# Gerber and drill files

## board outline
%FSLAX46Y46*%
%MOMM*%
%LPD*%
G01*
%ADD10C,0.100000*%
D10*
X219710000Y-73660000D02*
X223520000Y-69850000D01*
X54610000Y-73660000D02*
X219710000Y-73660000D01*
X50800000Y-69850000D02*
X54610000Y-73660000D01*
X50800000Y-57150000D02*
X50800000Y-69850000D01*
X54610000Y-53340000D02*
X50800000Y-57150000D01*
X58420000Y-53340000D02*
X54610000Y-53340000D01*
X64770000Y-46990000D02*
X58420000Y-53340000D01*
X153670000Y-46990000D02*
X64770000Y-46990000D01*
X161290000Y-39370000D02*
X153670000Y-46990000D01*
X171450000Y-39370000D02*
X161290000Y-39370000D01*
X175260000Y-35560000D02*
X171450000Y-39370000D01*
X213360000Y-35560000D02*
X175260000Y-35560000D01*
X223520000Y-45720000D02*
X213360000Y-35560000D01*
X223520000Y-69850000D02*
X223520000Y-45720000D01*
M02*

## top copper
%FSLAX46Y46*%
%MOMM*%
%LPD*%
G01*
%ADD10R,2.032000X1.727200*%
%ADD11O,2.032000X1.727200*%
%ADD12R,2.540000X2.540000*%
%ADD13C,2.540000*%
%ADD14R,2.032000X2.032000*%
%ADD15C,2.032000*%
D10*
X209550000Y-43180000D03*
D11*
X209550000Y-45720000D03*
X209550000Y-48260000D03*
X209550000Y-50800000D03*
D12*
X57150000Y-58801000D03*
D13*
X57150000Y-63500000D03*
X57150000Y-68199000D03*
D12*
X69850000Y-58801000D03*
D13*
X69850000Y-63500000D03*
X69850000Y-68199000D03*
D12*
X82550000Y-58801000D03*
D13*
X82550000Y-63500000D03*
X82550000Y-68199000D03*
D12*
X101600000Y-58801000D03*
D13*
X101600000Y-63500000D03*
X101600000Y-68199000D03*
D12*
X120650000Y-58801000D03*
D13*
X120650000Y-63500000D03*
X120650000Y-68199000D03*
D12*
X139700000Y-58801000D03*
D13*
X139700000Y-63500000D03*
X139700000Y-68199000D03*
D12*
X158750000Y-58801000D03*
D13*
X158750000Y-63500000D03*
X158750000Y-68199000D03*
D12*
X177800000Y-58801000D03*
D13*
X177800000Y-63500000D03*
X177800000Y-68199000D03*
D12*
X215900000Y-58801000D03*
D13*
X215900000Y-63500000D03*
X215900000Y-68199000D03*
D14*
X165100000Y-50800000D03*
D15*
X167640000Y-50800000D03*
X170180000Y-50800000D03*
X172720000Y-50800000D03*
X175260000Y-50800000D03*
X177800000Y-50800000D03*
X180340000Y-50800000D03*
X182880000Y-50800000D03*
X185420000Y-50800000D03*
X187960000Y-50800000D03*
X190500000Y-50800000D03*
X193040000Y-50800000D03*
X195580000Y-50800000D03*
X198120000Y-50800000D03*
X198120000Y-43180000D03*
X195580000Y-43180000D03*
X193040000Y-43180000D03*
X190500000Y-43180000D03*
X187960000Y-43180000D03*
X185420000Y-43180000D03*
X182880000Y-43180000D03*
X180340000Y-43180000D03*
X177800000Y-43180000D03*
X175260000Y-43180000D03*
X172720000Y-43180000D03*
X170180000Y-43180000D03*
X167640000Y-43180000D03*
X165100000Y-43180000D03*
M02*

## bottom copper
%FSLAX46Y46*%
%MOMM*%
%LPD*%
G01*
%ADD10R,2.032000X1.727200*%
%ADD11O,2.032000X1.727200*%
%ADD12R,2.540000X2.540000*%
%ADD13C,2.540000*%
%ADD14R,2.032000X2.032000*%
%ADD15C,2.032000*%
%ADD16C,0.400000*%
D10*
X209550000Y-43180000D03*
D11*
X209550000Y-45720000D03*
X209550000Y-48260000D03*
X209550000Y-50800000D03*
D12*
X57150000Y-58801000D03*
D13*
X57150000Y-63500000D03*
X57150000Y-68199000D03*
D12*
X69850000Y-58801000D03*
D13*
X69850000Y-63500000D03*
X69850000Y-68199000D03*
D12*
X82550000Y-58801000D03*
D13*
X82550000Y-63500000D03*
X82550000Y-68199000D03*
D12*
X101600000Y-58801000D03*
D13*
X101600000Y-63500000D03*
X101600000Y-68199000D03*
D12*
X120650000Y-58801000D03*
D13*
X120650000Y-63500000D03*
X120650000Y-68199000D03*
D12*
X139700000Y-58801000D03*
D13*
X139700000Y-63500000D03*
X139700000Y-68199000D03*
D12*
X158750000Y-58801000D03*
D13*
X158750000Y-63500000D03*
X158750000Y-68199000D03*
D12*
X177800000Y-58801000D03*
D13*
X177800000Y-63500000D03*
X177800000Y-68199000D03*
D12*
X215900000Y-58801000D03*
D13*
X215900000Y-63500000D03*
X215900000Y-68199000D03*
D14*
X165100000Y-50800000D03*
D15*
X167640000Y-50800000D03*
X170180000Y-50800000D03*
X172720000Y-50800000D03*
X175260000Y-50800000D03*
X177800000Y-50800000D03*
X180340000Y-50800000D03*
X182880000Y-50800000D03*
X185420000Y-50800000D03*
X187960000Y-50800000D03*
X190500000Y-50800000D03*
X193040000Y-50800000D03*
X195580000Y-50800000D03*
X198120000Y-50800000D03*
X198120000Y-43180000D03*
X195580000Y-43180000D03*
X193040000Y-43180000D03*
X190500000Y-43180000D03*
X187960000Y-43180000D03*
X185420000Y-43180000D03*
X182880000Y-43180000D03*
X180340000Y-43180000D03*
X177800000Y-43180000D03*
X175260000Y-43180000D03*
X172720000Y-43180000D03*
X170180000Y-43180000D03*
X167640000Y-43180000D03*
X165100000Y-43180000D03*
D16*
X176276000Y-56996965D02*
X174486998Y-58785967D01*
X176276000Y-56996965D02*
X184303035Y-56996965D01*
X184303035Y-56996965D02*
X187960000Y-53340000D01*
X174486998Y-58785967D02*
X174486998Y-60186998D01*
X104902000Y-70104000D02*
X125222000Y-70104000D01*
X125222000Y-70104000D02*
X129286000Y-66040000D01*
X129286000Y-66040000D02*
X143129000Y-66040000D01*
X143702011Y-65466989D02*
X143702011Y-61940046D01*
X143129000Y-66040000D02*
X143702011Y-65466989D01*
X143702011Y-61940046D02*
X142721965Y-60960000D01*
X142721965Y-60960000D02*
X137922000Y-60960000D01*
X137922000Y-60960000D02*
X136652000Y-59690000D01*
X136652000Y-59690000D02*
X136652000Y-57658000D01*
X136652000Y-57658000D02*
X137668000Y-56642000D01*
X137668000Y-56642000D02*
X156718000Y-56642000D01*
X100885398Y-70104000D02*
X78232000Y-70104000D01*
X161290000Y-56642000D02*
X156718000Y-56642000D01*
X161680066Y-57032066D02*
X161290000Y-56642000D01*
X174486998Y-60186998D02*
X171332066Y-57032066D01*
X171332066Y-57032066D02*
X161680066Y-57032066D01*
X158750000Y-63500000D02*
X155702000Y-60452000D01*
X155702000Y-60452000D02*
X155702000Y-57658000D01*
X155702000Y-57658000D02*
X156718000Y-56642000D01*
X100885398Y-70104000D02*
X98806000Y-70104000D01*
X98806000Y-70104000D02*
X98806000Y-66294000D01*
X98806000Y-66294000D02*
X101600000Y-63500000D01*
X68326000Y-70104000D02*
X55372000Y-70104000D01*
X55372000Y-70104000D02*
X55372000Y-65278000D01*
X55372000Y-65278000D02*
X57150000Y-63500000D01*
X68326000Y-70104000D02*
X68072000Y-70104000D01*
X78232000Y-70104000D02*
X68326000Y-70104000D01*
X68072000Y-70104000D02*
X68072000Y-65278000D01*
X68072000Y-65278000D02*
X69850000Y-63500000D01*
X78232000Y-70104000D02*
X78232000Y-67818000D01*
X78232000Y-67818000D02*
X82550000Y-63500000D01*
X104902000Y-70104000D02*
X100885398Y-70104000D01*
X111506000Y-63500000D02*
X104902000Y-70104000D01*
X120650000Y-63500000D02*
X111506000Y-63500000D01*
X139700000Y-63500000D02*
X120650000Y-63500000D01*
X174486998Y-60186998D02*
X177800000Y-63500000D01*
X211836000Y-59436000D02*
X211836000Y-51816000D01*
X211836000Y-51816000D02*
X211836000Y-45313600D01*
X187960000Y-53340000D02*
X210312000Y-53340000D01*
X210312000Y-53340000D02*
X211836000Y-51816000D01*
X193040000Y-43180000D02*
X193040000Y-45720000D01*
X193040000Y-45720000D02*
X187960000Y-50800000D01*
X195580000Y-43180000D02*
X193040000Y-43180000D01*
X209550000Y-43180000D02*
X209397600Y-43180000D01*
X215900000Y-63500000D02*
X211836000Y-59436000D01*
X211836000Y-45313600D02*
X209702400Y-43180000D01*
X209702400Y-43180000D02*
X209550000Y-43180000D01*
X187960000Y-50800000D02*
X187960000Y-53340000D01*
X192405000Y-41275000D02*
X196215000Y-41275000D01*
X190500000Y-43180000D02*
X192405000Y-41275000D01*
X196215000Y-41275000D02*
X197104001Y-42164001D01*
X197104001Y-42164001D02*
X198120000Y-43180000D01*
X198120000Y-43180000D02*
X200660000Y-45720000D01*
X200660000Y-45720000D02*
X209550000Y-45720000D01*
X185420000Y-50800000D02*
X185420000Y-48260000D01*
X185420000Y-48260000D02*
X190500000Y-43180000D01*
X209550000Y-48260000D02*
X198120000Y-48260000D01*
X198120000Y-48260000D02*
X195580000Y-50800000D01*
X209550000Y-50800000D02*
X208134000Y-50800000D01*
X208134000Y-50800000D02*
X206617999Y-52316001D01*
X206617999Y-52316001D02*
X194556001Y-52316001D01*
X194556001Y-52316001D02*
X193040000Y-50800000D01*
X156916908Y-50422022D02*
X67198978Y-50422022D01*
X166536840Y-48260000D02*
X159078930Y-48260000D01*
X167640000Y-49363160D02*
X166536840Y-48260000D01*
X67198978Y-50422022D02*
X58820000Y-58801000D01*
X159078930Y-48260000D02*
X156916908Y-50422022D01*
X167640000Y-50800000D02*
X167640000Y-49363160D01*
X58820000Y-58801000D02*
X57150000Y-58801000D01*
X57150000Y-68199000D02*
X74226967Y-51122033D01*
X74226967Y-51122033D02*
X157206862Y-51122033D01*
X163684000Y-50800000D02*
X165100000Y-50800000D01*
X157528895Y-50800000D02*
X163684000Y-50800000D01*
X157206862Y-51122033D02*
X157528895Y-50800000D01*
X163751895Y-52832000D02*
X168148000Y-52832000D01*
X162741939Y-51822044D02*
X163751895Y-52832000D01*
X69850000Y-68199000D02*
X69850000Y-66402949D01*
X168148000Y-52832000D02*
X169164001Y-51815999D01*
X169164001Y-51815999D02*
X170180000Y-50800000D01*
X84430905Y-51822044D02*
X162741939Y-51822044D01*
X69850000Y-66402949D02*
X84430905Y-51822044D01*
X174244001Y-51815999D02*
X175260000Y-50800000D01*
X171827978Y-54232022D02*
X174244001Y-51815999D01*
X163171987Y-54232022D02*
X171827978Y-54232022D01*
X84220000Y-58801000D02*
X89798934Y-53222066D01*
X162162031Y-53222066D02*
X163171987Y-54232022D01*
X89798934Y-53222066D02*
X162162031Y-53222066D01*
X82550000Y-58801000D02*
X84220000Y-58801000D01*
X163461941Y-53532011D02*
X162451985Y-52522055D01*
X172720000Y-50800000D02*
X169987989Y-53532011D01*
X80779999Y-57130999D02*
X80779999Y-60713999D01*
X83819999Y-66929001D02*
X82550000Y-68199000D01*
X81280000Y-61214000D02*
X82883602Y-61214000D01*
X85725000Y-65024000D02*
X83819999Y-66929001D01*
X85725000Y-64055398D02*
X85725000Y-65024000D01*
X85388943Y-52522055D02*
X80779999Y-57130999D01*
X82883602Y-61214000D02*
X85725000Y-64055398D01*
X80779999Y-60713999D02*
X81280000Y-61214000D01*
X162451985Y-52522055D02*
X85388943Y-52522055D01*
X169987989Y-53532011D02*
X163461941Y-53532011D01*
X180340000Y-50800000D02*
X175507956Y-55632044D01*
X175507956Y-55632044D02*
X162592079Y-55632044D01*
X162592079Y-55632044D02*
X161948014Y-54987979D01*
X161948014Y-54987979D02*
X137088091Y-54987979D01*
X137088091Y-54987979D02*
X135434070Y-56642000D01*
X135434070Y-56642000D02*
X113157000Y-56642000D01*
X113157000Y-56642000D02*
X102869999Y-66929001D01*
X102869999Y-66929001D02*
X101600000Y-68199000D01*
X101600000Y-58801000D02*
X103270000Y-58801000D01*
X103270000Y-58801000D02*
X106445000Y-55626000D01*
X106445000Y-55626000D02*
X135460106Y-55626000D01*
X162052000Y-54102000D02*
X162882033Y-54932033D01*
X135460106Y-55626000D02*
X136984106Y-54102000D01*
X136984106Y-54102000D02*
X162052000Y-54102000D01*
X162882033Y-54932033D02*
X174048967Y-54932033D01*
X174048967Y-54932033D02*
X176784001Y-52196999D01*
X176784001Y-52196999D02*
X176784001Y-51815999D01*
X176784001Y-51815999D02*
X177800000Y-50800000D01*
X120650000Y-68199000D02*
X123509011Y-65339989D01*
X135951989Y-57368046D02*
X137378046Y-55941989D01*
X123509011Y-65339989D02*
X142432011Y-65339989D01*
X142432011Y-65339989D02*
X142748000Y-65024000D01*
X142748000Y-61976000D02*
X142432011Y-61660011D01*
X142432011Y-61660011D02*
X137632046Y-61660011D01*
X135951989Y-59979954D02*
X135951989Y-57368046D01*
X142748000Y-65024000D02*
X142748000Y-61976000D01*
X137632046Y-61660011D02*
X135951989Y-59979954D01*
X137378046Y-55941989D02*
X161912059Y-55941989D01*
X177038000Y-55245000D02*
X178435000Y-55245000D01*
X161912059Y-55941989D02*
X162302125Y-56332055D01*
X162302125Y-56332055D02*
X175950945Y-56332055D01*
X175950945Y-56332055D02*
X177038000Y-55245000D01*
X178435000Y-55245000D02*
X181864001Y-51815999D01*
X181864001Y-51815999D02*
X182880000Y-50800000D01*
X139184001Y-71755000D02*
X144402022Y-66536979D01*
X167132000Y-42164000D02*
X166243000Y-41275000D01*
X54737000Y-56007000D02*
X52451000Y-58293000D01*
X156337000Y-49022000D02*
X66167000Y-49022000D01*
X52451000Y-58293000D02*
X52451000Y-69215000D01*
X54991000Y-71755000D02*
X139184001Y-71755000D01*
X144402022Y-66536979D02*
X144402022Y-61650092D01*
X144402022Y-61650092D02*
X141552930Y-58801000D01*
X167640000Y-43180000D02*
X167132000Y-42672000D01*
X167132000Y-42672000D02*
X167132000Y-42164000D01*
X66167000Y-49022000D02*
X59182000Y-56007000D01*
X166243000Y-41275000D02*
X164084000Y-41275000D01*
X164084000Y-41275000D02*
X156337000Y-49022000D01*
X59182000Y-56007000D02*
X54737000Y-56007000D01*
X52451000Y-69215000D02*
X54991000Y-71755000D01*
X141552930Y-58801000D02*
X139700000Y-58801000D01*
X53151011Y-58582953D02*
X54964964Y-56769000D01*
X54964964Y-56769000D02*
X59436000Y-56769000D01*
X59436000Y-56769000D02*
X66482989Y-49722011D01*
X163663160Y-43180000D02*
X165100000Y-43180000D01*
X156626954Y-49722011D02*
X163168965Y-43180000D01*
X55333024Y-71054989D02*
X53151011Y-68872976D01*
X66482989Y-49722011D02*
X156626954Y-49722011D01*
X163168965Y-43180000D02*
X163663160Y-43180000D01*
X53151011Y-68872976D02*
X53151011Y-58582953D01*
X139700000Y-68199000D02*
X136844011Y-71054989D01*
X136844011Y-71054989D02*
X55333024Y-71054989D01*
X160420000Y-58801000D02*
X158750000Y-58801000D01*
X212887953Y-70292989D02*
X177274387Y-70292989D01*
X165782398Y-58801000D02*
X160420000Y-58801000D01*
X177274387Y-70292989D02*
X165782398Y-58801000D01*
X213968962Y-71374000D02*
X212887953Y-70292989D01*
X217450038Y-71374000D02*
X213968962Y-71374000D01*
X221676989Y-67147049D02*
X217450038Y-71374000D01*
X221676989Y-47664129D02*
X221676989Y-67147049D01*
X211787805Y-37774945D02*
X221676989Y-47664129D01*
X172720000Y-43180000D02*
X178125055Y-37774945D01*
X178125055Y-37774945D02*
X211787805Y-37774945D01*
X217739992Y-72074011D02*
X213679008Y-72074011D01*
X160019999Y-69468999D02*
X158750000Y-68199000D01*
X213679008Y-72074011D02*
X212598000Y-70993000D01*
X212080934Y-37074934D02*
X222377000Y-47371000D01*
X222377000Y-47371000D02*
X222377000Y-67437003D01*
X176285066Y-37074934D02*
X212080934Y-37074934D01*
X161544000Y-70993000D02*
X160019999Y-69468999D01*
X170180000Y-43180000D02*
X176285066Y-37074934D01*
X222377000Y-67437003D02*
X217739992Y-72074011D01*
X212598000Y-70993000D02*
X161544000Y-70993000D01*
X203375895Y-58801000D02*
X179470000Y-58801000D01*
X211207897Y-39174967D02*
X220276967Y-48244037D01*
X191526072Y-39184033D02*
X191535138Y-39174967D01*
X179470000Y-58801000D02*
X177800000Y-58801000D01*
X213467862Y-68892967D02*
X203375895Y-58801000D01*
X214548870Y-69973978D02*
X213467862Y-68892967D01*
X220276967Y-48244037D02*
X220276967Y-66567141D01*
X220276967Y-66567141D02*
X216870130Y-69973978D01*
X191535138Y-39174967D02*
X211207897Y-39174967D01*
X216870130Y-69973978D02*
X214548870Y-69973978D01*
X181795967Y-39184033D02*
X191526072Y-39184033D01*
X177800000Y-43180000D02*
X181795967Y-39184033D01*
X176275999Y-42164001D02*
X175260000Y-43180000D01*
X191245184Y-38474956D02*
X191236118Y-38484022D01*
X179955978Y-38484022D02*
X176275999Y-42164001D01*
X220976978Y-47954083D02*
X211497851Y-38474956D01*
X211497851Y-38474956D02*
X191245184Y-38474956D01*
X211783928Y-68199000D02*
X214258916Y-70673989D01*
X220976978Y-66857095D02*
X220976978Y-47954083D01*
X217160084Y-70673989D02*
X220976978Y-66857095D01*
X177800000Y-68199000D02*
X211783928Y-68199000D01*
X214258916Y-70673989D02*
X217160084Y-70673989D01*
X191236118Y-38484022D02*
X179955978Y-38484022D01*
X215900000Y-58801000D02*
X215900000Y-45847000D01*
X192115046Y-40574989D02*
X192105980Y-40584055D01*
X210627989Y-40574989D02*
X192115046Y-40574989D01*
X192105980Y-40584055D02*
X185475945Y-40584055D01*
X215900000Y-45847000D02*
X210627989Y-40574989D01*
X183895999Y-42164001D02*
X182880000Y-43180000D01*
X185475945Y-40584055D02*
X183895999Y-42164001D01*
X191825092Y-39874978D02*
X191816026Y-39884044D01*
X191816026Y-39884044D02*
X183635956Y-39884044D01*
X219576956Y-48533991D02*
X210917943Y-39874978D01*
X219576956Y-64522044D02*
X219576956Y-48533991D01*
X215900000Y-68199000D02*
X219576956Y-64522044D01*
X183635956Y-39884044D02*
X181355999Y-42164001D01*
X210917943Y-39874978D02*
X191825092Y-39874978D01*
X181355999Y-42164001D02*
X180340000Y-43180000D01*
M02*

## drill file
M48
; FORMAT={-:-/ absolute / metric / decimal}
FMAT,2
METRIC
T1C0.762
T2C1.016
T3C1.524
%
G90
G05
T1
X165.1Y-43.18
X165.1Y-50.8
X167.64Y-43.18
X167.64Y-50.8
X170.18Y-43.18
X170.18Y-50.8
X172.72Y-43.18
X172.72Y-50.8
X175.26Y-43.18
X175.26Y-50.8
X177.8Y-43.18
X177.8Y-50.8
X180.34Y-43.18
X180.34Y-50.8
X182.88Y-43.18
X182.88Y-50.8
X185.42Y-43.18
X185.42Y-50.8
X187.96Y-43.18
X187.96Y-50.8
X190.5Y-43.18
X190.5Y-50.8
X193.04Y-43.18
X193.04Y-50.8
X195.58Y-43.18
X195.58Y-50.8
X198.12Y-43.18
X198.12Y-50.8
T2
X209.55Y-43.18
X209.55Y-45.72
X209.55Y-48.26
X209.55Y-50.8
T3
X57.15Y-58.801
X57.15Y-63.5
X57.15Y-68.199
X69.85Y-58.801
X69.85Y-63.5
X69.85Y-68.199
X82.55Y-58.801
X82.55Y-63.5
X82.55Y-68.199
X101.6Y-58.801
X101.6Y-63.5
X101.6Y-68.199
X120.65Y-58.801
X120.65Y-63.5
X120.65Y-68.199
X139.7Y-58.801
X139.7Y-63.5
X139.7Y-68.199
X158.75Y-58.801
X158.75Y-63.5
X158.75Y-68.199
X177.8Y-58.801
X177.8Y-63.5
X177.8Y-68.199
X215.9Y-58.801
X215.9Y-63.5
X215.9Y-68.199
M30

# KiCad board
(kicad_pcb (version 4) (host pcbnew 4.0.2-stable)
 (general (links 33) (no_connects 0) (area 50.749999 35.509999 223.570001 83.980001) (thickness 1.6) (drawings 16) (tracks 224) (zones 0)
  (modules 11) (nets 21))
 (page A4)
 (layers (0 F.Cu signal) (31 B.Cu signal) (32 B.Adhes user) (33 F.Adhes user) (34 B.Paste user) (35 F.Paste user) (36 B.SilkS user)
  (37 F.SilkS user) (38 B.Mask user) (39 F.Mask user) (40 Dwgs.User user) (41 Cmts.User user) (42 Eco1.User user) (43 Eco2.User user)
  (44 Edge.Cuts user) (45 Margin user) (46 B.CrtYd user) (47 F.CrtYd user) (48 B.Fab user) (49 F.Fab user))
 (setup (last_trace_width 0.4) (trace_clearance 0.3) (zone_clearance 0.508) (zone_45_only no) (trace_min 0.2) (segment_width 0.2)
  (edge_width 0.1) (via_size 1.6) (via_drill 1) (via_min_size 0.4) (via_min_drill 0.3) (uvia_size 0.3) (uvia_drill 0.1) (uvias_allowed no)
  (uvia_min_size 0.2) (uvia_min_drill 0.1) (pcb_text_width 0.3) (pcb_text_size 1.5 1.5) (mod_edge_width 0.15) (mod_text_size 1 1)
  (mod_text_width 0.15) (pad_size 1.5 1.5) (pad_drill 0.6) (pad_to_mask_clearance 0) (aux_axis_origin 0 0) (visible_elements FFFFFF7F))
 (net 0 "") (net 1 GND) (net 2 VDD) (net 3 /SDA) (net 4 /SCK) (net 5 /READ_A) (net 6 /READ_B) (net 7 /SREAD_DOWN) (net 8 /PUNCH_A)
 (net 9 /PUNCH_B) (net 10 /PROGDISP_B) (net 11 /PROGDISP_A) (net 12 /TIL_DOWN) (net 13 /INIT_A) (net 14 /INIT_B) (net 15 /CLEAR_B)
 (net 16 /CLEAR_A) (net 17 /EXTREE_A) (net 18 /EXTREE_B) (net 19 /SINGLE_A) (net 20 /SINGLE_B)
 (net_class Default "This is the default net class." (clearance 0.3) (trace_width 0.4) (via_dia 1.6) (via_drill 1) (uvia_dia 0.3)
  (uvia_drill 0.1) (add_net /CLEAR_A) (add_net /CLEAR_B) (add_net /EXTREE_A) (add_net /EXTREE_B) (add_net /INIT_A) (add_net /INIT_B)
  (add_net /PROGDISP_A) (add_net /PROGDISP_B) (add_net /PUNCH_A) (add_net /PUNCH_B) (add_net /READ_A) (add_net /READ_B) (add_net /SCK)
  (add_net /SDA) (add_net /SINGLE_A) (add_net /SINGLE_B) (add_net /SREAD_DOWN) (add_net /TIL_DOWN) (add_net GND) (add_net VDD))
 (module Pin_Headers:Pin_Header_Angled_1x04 (layer F.Cu) (at 209.55 43.18)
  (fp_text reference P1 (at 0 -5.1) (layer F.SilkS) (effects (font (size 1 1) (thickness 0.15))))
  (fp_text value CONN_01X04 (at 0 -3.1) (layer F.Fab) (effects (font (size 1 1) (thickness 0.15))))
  (pad 1 thru_hole rect (at 0 0) (size 2.032 1.7272) (drill 1.016) (layers *.Cu *.Mask F.SilkS) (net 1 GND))
  (pad 2 thru_hole oval (at 0 2.54) (size 2.032 1.7272) (drill 1.016) (layers *.Cu *.Mask F.SilkS) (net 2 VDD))
  (pad 3 thru_hole oval (at 0 5.08) (size 2.032 1.7272) (drill 1.016) (layers *.Cu *.Mask F.SilkS) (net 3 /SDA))
  (pad 4 thru_hole oval (at 0 7.62) (size 2.032 1.7272) (drill 1.016) (layers *.Cu *.Mask F.SilkS) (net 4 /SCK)))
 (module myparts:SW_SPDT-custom (layer F.Cu) (at 57.15 63.5 270)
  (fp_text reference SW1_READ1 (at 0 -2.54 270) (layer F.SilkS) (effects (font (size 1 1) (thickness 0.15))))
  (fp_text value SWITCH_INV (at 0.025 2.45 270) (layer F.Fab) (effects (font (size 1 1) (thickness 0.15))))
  (pad 1 thru_hole rect (at -4.699 0 270) (size 2.54 2.54) (drill 1.524) (layers *.Cu *.Mask F.SilkS) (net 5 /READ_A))
  (pad 2 thru_hole circle (at 0 0 270) (size 2.54 2.54) (drill 1.524) (layers *.Cu *.Mask F.SilkS) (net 1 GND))
  (pad 3 thru_hole circle (at 4.699 0 270) (size 2.54 2.54) (drill 1.524) (layers *.Cu *.Mask F.SilkS) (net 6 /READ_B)))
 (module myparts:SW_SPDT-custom (layer F.Cu) (at 69.85 63.5 270)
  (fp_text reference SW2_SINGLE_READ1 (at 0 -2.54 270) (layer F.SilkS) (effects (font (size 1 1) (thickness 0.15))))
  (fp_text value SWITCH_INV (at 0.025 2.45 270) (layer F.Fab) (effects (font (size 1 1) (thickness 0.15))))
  (pad 1 thru_hole rect (at -4.699 0 270) (size 2.54 2.54) (drill 1.524) (layers *.Cu *.Mask F.SilkS))
  (pad 2 thru_hole circle (at 0 0 270) (size 2.54 2.54) (drill 1.524) (layers *.Cu *.Mask F.SilkS) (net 1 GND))
  (pad 3 thru_hole circle (at 4.699 0 270) (size 2.54 2.54) (drill 1.524) (layers *.Cu *.Mask F.SilkS) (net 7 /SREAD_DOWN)))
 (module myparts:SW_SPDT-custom (layer F.Cu) (at 82.55 63.5 270)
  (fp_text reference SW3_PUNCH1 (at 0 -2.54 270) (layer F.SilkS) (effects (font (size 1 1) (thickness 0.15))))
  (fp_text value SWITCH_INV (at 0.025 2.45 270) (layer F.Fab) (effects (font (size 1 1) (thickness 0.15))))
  (pad 1 thru_hole rect (at -4.699 0 270) (size 2.54 2.54) (drill 1.524) (layers *.Cu *.Mask F.SilkS) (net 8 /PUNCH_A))
  (pad 2 thru_hole circle (at 0 0 270) (size 2.54 2.54) (drill 1.524) (layers *.Cu *.Mask F.SilkS) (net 1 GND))
  (pad 3 thru_hole circle (at 4.699 0 270) (size 2.54 2.54) (drill 1.524) (layers *.Cu *.Mask F.SilkS) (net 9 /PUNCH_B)))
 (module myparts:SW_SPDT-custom (layer F.Cu) (at 101.6 63.5 270)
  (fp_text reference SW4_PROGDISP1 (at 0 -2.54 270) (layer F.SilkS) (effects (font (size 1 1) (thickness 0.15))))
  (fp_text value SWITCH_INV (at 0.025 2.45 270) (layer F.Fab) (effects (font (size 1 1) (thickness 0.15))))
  (pad 1 thru_hole rect (at -4.699 0 270) (size 2.54 2.54) (drill 1.524) (layers *.Cu *.Mask F.SilkS) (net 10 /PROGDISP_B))
  (pad 2 thru_hole circle (at 0 0 270) (size 2.54 2.54) (drill 1.524) (layers *.Cu *.Mask F.SilkS) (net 1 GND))
  (pad 3 thru_hole circle (at 4.699 0 270) (size 2.54 2.54) (drill 1.524) (layers *.Cu *.Mask F.SilkS) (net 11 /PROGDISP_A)))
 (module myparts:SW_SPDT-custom (layer F.Cu) (at 120.65 63.5 270)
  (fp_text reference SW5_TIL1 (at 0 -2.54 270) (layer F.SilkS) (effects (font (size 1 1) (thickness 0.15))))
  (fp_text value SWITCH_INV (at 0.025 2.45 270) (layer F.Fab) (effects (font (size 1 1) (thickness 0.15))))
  (pad 1 thru_hole rect (at -4.699 0 270) (size 2.54 2.54) (drill 1.524) (layers *.Cu *.Mask F.SilkS))
  (pad 2 thru_hole circle (at 0 0 270) (size 2.54 2.54) (drill 1.524) (layers *.Cu *.Mask F.SilkS) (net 1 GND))
  (pad 3 thru_hole circle (at 4.699 0 270) (size 2.54 2.54) (drill 1.524) (layers *.Cu *.Mask F.SilkS) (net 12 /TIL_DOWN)))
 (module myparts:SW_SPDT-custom (layer F.Cu) (at 139.7 63.5 270)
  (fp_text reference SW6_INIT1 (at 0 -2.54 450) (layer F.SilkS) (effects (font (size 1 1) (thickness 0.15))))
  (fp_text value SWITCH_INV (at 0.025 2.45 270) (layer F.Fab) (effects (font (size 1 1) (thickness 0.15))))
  (pad 1 thru_hole rect (at -4.699 0 270) (size 2.54 2.54) (drill 1.524) (layers *.Cu *.Mask F.SilkS) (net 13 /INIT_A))
  (pad 2 thru_hole circle (at 0 0 270) (size 2.54 2.54) (drill 1.524) (layers *.Cu *.Mask F.SilkS) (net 1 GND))
  (pad 3 thru_hole circle (at 4.699 0 270) (size 2.54 2.54) (drill 1.524) (layers *.Cu *.Mask F.SilkS) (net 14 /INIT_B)))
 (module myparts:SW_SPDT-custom (layer F.Cu) (at 158.75 63.5 270)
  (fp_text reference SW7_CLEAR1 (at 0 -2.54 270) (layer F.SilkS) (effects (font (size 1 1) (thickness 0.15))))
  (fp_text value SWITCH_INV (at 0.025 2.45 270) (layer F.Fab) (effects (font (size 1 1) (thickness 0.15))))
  (pad 1 thru_hole rect (at -4.699 0 270) (size 2.54 2.54) (drill 1.524) (layers *.Cu *.Mask F.SilkS) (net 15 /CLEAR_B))
  (pad 2 thru_hole circle (at 0 0 270) (size 2.54 2.54) (drill 1.524) (layers *.Cu *.Mask F.SilkS) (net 1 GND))
  (pad 3 thru_hole circle (at 4.699 0 270) (size 2.54 2.54) (drill 1.524) (layers *.Cu *.Mask F.SilkS) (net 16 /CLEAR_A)))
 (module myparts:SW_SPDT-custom (layer F.Cu) (at 177.8 63.5 270)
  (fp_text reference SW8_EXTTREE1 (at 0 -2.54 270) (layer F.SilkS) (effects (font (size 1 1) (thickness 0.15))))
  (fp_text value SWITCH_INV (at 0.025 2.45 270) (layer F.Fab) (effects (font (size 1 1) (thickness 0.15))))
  (pad 1 thru_hole rect (at -4.699 0 270) (size 2.54 2.54) (drill 1.524) (layers *.Cu *.Mask F.SilkS) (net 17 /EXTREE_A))
  (pad 2 thru_hole circle (at 0 0 270) (size 2.54 2.54) (drill 1.524) (layers *.Cu *.Mask F.SilkS) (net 1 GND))
  (pad 3 thru_hole circle (at 4.699 0 270) (size 2.54 2.54) (drill 1.524) (layers *.Cu *.Mask F.SilkS) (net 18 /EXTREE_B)))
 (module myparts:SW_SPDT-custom (layer F.Cu) (at 215.9 63.5 270)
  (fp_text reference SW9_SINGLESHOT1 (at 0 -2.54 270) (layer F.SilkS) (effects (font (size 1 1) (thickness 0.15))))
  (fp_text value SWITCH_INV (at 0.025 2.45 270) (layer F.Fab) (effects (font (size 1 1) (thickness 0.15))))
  (pad 1 thru_hole rect (at -4.699 0 270) (size 2.54 2.54) (drill 1.524) (layers *.Cu *.Mask F.SilkS) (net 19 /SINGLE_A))
  (pad 2 thru_hole circle (at 0 0 270) (size 2.54 2.54) (drill 1.524) (layers *.Cu *.Mask F.SilkS) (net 1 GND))
  (pad 3 thru_hole circle (at 4.699 0 270) (size 2.54 2.54) (drill 1.524) (layers *.Cu *.Mask F.SilkS) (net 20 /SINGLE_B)))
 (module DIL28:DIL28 (layer F.Cu) (at 165.1 50.8)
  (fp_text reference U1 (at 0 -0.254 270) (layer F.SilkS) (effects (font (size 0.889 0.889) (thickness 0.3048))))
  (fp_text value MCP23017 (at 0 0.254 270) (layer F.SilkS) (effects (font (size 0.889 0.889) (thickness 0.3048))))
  (pad 1 thru_hole rect (at 0 0) (size 2.032 2.032) (drill 0.762) (layers *.Cu *.Mask F.SilkS) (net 6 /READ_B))
  (pad 2 thru_hole circle (at 2.54 0) (size 2.032 2.032) (drill 0.762) (layers *.Cu *.Mask F.SilkS) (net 5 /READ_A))
  (pad 3 thru_hole circle (at 5.08 0) (size 2.032 2.032) (drill 0.762) (layers *.Cu *.Mask F.SilkS) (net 7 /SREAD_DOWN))
  (pad 4 thru_hole circle (at 7.62 0) (size 2.032 2.032) (drill 0.762) (layers *.Cu *.Mask F.SilkS) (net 9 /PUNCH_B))
  (pad 5 thru_hole circle (at 10.16 0) (size 2.032 2.032) (drill 0.762) (layers *.Cu *.Mask F.SilkS) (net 8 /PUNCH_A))
  (pad 6 thru_hole circle (at 12.7 0) (size 2.032 2.032) (drill 0.762) (layers *.Cu *.Mask F.SilkS) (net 10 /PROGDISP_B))
  (pad 7 thru_hole circle (at 15.24 0) (size 2.032 2.032) (drill 0.762) (layers *.Cu *.Mask F.SilkS) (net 11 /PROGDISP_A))
  (pad 8 thru_hole circle (at 17.78 0) (size 2.032 2.032) (drill 0.762) (layers *.Cu *.Mask F.SilkS) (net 12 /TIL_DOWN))
  (pad 9 thru_hole circle (at 20.32 0) (size 2.032 2.032) (drill 0.762) (layers *.Cu *.Mask F.SilkS) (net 2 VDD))
  (pad 10 thru_hole circle (at 22.86 0) (size 2.032 2.032) (drill 0.762) (layers *.Cu *.Mask F.SilkS) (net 1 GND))
  (pad 11 thru_hole circle (at 25.4 0) (size 2.032 2.032) (drill 0.762) (layers *.Cu *.Mask F.SilkS))
  (pad 12 thru_hole circle (at 27.94 0) (size 2.032 2.032) (drill 0.762) (layers *.Cu *.Mask F.SilkS) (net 4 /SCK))
  (pad 13 thru_hole circle (at 30.48 0) (size 2.032 2.032) (drill 0.762) (layers *.Cu *.Mask F.SilkS) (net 3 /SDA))
  (pad 14 thru_hole circle (at 33.02 0) (size 2.032 2.032) (drill 0.762) (layers *.Cu *.Mask F.SilkS))
  (pad 15 thru_hole circle (at 33.02 -7.62 180) (size 2.032 2.032) (drill 0.762) (layers *.Cu *.Mask F.SilkS) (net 2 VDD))
  (pad 16 thru_hole circle (at 30.48 -7.62 180) (size 2.032 2.032) (drill 0.762) (layers *.Cu *.Mask F.SilkS) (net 1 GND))
  (pad 17 thru_hole circle (at 27.94 -7.62 180) (size 2.032 2.032) (drill 0.762) (layers *.Cu *.Mask F.SilkS) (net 1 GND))
  (pad 18 thru_hole circle (at 25.4 -7.62 180) (size 2.032 2.032) (drill 0.762) (layers *.Cu *.Mask F.SilkS) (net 2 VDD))
  (pad 19 thru_hole circle (at 22.86 -7.62 180) (size 2.032 2.032) (drill 0.762) (layers *.Cu *.Mask F.SilkS))
  (pad 20 thru_hole circle (at 20.32 -7.62 180) (size 2.032 2.032) (drill 0.762) (layers *.Cu *.Mask F.SilkS))
  (pad 21 thru_hole circle (at 17.78 -7.62 180) (size 2.032 2.032) (drill 0.762) (layers *.Cu *.Mask F.SilkS) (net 19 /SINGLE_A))
  (pad 22 thru_hole circle (at 15.24 -7.62 180) (size 2.032 2.032) (drill 0.762) (layers *.Cu *.Mask F.SilkS) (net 20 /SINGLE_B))
  (pad 23 thru_hole circle (at 12.7 -7.62 180) (size 2.032 2.032) (drill 0.762) (layers *.Cu *.Mask F.SilkS) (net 17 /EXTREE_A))
  (pad 24 thru_hole circle (at 10.16 -7.62 180) (size 2.032 2.032) (drill 0.762) (layers *.Cu *.Mask F.SilkS) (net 18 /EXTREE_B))
  (pad 25 thru_hole circle (at 7.62 -7.62 180) (size 2.032 2.032) (drill 0.762) (layers *.Cu *.Mask F.SilkS) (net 15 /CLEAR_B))
  (pad 26 thru_hole circle (at 5.08 -7.62 180) (size 2.032 2.032) (drill 0.762) (layers *.Cu *.Mask F.SilkS) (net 16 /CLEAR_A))
  (pad 27 thru_hole circle (at 2.54 -7.62 180) (size 2.032 2.032) (drill 0.762) (layers *.Cu *.Mask F.SilkS) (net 13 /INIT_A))
  (pad 28 thru_hole circle (at 0 -7.62 180) (size 2.032 2.032) (drill 0.762) (layers *.Cu *.Mask F.SilkS) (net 14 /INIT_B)))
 (gr_line (start 219.71 73.66) (end 223.52 69.85) (layer Edge.Cuts) (width 0.1))
 (gr_line (start 54.61 73.66) (end 219.71 73.66) (layer Edge.Cuts) (width 0.1))
 (gr_line (start 50.8 69.85) (end 54.61 73.66) (layer Edge.Cuts) (width 0.1))
 (gr_line (start 50.8 57.15) (end 50.8 69.85) (layer Edge.Cuts) (width 0.1))
 (gr_line (start 54.61 53.34) (end 50.8 57.15) (layer Edge.Cuts) (width 0.1))
 (gr_line (start 58.42 53.34) (end 54.61 53.34) (layer Edge.Cuts) (width 0.1))
 (gr_line (start 64.77 46.99) (end 58.42 53.34) (layer Edge.Cuts) (width 0.1))
 (gr_line (start 153.67 46.99) (end 64.77 46.99) (layer Edge.Cuts) (width 0.1))
 (gr_line (start 161.29 39.37) (end 153.67 46.99) (layer Edge.Cuts) (width 0.1))
 (gr_line (start 171.45 39.37) (end 161.29 39.37) (layer Edge.Cuts) (width 0.1))
 (gr_line (start 175.26 35.56) (end 171.45 39.37) (layer Edge.Cuts) (width 0.1))
 (gr_line (start 213.36 35.56) (end 175.26 35.56) (layer Edge.Cuts) (width 0.1))
 (gr_line (start 223.52 45.72) (end 213.36 35.56) (layer Edge.Cuts) (width 0.1))
 (gr_line (start 223.52 69.85) (end 223.52 45.72) (layer Edge.Cuts) (width 0.1))
 (segment (start 176.276 56.996965) (end 174.486998 58.785967) (width 0.4) (layer B.Cu) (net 1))
 (segment (start 176.276 56.996965) (end 184.303035 56.996965) (width 0.4) (layer B.Cu) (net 1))
 (segment (start 184.303035 56.996965) (end 187.96 53.34) (width 0.4) (layer B.Cu) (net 1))
 (segment (start 174.486998 58.785967) (end 174.486998 60.186998) (width 0.4) (layer B.Cu) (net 1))
 (segment (start 104.902 70.104) (end 125.222 70.104) (width 0.4) (layer B.Cu) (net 1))
 (segment (start 125.222 70.104) (end 129.286 66.04) (width 0.4) (layer B.Cu) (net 1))
 (segment (start 129.286 66.04) (end 143.129 66.04) (width 0.4) (layer B.Cu) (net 1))
 (segment (start 143.702011 65.466989) (end 143.702011 61.940046) (width 0.4) (layer B.Cu) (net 1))
 (segment (start 143.129 66.04) (end 143.702011 65.466989) (width 0.4) (layer B.Cu) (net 1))
 (segment (start 143.702011 61.940046) (end 142.721965 60.96) (width 0.4) (layer B.Cu) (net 1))
 (segment (start 142.721965 60.96) (end 137.922 60.96) (width 0.4) (layer B.Cu) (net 1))
 (segment (start 137.922 60.96) (end 136.652 59.69) (width 0.4) (layer B.Cu) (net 1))
 (segment (start 136.652 59.69) (end 136.652 57.658) (width 0.4) (layer B.Cu) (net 1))
 (segment (start 136.652 57.658) (end 137.668 56.642) (width 0.4) (layer B.Cu) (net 1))
 (segment (start 137.668 56.642) (end 156.718 56.642) (width 0.4) (layer B.Cu) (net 1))
 (segment (start 100.885398 70.104) (end 78.232 70.104) (width 0.4) (layer B.Cu) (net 1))
 (segment (start 161.29 56.642) (end 156.718 56.642) (width 0.4) (layer B.Cu) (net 1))
 (segment (start 161.680066 57.032066) (end 161.29 56.642) (width 0.4) (layer B.Cu) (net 1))
 (segment (start 174.486998 60.186998) (end 171.332066 57.032066) (width 0.4) (layer B.Cu) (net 1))
 (segment (start 171.332066 57.032066) (end 161.680066 57.032066) (width 0.4) (layer B.Cu) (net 1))
 (segment (start 158.75 63.5) (end 155.702 60.452) (width 0.4) (layer B.Cu) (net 1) (status 10))
 (segment (start 155.702 60.452) (end 155.702 57.658) (width 0.4) (layer B.Cu) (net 1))
 (segment (start 155.702 57.658) (end 156.718 56.642) (width 0.4) (layer B.Cu) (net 1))
 (segment (start 100.885398 70.104) (end 98.806 70.104) (width 0.4) (layer B.Cu) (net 1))
 (segment (start 98.806 70.104) (end 98.806 66.294) (width 0.4) (layer B.Cu) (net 1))
 (segment (start 98.806 66.294) (end 101.6 63.5) (width 0.4) (layer B.Cu) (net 1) (status 20))
 (segment (start 68.326 70.104) (end 55.372 70.104) (width 0.4) (layer B.Cu) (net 1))
 (segment (start 55.372 70.104) (end 55.372 65.278) (width 0.4) (layer B.Cu) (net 1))
 (segment (start 55.372 65.278) (end 57.15 63.5) (width 0.4) (layer B.Cu) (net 1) (status 20))
 (segment (start 68.326 70.104) (end 68.072 70.104) (width 0.4) (layer B.Cu) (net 1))
 (segment (start 78.232 70.104) (end 68.326 70.104) (width 0.4) (layer B.Cu) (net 1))
 (segment (start 68.072 70.104) (end 68.072 65.278) (width 0.4) (layer B.Cu) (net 1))
 (segment (start 68.072 65.278) (end 69.85 63.5) (width 0.4) (layer B.Cu) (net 1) (status 20))
 (segment (start 78.232 70.104) (end 78.232 67.818) (width 0.4) (layer B.Cu) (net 1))
 (segment (start 78.232 67.818) (end 82.55 63.5) (width 0.4) (layer B.Cu) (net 1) (status 20))
 (segment (start 104.902 70.104) (end 100.885398 70.104) (width 0.4) (layer B.Cu) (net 1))
 (segment (start 111.506 63.5) (end 104.902 70.104) (width 0.4) (layer B.Cu) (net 1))
 (segment (start 120.65 63.5) (end 111.506 63.5) (width 0.4) (layer B.Cu) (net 1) (status 10))
 (segment (start 139.7 63.5) (end 120.65 63.5) (width 0.4) (layer B.Cu) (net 1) (status 30))
 (segment (start 174.486998 60.186998) (end 177.8 63.5) (width 0.4) (layer B.Cu) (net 1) (status 20))
 (segment (start 211.836 59.436) (end 211.836 51.816) (width 0.4) (layer B.Cu) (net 1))
 (segment (start 211.836 51.816) (end 211.836 45.3136) (width 0.4) (layer B.Cu) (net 1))
 (segment (start 187.96 53.34) (end 210.312 53.34) (width 0.4) (layer B.Cu) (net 1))
 (segment (start 210.312 53.34) (end 211.836 51.816) (width 0.4) (layer B.Cu) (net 1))
 (segment (start 193.04 43.18) (end 193.04 45.72) (width 0.4) (layer B.Cu) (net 1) (status 10))
 (segment (start 193.04 45.72) (end 187.96 50.8) (width 0.4) (layer B.Cu) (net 1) (status 20))
 (segment (start 195.58 43.18) (end 193.04 43.18) (width 0.4) (layer B.Cu) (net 1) (status 30))
 (segment (start 209.55 43.18) (end 209.3976 43.18) (width 0.4) (layer B.Cu) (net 1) (status 30))
 (segment (start 215.9 63.5) (end 211.836 59.436) (width 0.4) (layer B.Cu) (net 1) (status 10))
 (segment (start 211.836 45.3136) (end 209.7024 43.18) (width 0.4) (layer B.Cu) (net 1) (status 20))
 (segment (start 209.7024 43.18) (end 209.55 43.18) (width 0.4) (layer B.Cu) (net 1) (status 30))
 (segment (start 187.96 50.8) (end 187.96 53.34) (width 0.4) (layer B.Cu) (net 1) (status 10))
 (segment (start 192.405 41.275) (end 196.215 41.275) (width 0.4) (layer B.Cu) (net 2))
 (segment (start 190.5 43.18) (end 192.405 41.275) (width 0.4) (layer B.Cu) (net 2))
 (segment (start 196.215 41.275) (end 197.104001 42.164001) (width 0.4) (layer B.Cu) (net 2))
 (segment (start 197.104001 42.164001) (end 198.12 43.18) (width 0.4) (layer B.Cu) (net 2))
 (segment (start 198.12 43.18) (end 200.66 45.72) (width 0.4) (layer B.Cu) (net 2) (status 10))
 (segment (start 200.66 45.72) (end 209.55 45.72) (width 0.4) (layer B.Cu) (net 2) (status 20))
 (segment (start 185.42 50.8) (end 185.42 48.26) (width 0.4) (layer B.Cu) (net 2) (status 10))
 (segment (start 185.42 48.26) (end 190.5 43.18) (width 0.4) (layer B.Cu) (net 2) (status 20))
 (segment (start 209.55 48.26) (end 198.12 48.26) (width 0.4) (layer B.Cu) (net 3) (status 10))
 (segment (start 198.12 48.26) (end 195.58 50.8) (width 0.4) (layer B.Cu) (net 3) (status 20))
 (segment (start 209.55 50.8) (end 208.134 50.8) (width 0.4) (layer B.Cu) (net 4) (status 10))
 (segment (start 208.134 50.8) (end 206.617999 52.316001) (width 0.4) (layer B.Cu) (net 4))
 (segment (start 206.617999 52.316001) (end 194.556001 52.316001) (width 0.4) (layer B.Cu) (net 4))
 (segment (start 194.556001 52.316001) (end 193.04 50.8) (width 0.4) (layer B.Cu) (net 4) (status 20))
 (segment (start 156.916908 50.422022) (end 67.198978 50.422022) (width 0.4) (layer B.Cu) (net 5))
 (segment (start 166.53684 48.26) (end 159.07893 48.26) (width 0.4) (layer B.Cu) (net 5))
 (segment (start 167.64 49.36316) (end 166.53684 48.26) (width 0.4) (layer B.Cu) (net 5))
 (segment (start 67.198978 50.422022) (end 58.82 58.801) (width 0.4) (layer B.Cu) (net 5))
 (segment (start 159.07893 48.26) (end 156.916908 50.422022) (width 0.4) (layer B.Cu) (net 5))
 (segment (start 167.64 50.8) (end 167.64 49.36316) (width 0.4) (layer B.Cu) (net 5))
 (segment (start 58.82 58.801) (end 57.15 58.801) (width 0.4) (layer B.Cu) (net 5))
 (segment (start 57.15 68.199) (end 74.226967 51.122033) (width 0.4) (layer B.Cu) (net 6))
 (segment (start 74.226967 51.122033) (end 157.206862 51.122033) (width 0.4) (layer B.Cu) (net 6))
 (segment (start 163.684 50.8) (end 165.1 50.8) (width 0.4) (layer B.Cu) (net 6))
 (segment (start 157.528895 50.8) (end 163.684 50.8) (width 0.4) (layer B.Cu) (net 6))
 (segment (start 157.206862 51.122033) (end 157.528895 50.8) (width 0.4) (layer B.Cu) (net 6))
 (segment (start 163.751895 52.832) (end 168.148 52.832) (width 0.4) (layer B.Cu) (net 7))
 (segment (start 162.741939 51.822044) (end 163.751895 52.832) (width 0.4) (layer B.Cu) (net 7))
 (segment (start 69.85 68.199) (end 69.85 66.402949) (width 0.4) (layer B.Cu) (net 7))
 (segment (start 168.148 52.832) (end 169.164001 51.815999) (width 0.4) (layer B.Cu) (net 7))
 (segment (start 169.164001 51.815999) (end 170.18 50.8) (width 0.4) (layer B.Cu) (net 7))
 (segment (start 84.430905 51.822044) (end 162.741939 51.822044) (width 0.4) (layer B.Cu) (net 7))
 (segment (start 69.85 66.402949) (end 84.430905 51.822044) (width 0.4) (layer B.Cu) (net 7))
 (segment (start 174.244001 51.815999) (end 175.26 50.8) (width 0.4) (layer B.Cu) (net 8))
 (segment (start 171.827978 54.232022) (end 174.244001 51.815999) (width 0.4) (layer B.Cu) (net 8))
 (segment (start 163.171987 54.232022) (end 171.827978 54.232022) (width 0.4) (layer B.Cu) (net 8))
 (segment (start 84.22 58.801) (end 89.798934 53.222066) (width 0.4) (layer B.Cu) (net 8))
 (segment (start 162.162031 53.222066) (end 163.171987 54.232022) (width 0.4) (layer B.Cu) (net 8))
 (segment (start 89.798934 53.222066) (end 162.162031 53.222066) (width 0.4) (layer B.Cu) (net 8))
 (segment (start 82.55 58.801) (end 84.22 58.801) (width 0.4) (layer B.Cu) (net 8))
 (segment (start 163.461941 53.532011) (end 162.451985 52.522055) (width 0.4) (layer B.Cu) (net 9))
 (segment (start 172.72 50.8) (end 169.987989 53.532011) (width 0.4) (layer B.Cu) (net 9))
 (segment (start 80.779999 57.130999) (end 80.779999 60.713999) (width 0.4) (layer B.Cu) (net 9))
 (segment (start 83.819999 66.929001) (end 82.55 68.199) (width 0.4) (layer B.Cu) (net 9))
 (segment (start 81.28 61.214) (end 82.883602 61.214) (width 0.4) (layer B.Cu) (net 9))
 (segment (start 85.725 65.024) (end 83.819999 66.929001) (width 0.4) (layer B.Cu) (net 9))
 (segment (start 85.725 64.055398) (end 85.725 65.024) (width 0.4) (layer B.Cu) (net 9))
 (segment (start 85.388943 52.522055) (end 80.779999 57.130999) (width 0.4) (layer B.Cu) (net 9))
 (segment (start 82.883602 61.214) (end 85.725 64.055398) (width 0.4) (layer B.Cu) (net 9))
 (segment (start 80.779999 60.713999) (end 81.28 61.214) (width 0.4) (layer B.Cu) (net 9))
 (segment (start 162.451985 52.522055) (end 85.388943 52.522055) (width 0.4) (layer B.Cu) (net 9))
 (segment (start 169.987989 53.532011) (end 163.461941 53.532011) (width 0.4) (layer B.Cu) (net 9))
 (segment (start 180.34 50.8) (end 175.507956 55.632044) (width 0.4) (layer B.Cu) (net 11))
 (segment (start 175.507956 55.632044) (end 162.592079 55.632044) (width 0.4) (layer B.Cu) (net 11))
 (segment (start 162.592079 55.632044) (end 161.948014 54.987979) (width 0.4) (layer B.Cu) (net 11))
 (segment (start 161.948014 54.987979) (end 137.088091 54.987979) (width 0.4) (layer B.Cu) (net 11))
 (segment (start 137.088091 54.987979) (end 135.43407 56.642) (width 0.4) (layer B.Cu) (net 11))
 (segment (start 135.43407 56.642) (end 113.157 56.642) (width 0.4) (layer B.Cu) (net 11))
 (segment (start 113.157 56.642) (end 102.869999 66.929001) (width 0.4) (layer B.Cu) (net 11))
 (segment (start 102.869999 66.929001) (end 101.6 68.199) (width 0.4) (layer B.Cu) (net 11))
 (segment (start 101.6 58.801) (end 103.27 58.801) (width 0.4) (layer B.Cu) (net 10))
 (segment (start 103.27 58.801) (end 106.445 55.626) (width 0.4) (layer B.Cu) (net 10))
 (segment (start 106.445 55.626) (end 135.460106 55.626) (width 0.4) (layer B.Cu) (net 10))
 (segment (start 162.052 54.102) (end 162.882033 54.932033) (width 0.4) (layer B.Cu) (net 10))
 (segment (start 135.460106 55.626) (end 136.984106 54.102) (width 0.4) (layer B.Cu) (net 10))
 (segment (start 136.984106 54.102) (end 162.052 54.102) (width 0.4) (layer B.Cu) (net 10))
 (segment (start 162.882033 54.932033) (end 174.048967 54.932033) (width 0.4) (layer B.Cu) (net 10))
 (segment (start 174.048967 54.932033) (end 176.784001 52.196999) (width 0.4) (layer B.Cu) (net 10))
 (segment (start 176.784001 52.196999) (end 176.784001 51.815999) (width 0.4) (layer B.Cu) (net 10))
 (segment (start 176.784001 51.815999) (end 177.8 50.8) (width 0.4) (layer B.Cu) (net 10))
 (segment (start 120.65 68.199) (end 123.509011 65.339989) (width 0.4) (layer B.Cu) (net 12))
 (segment (start 135.951989 57.368046) (end 137.378046 55.941989) (width 0.4) (layer B.Cu) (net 12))
 (segment (start 123.509011 65.339989) (end 142.432011 65.339989) (width 0.4) (layer B.Cu) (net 12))
 (segment (start 142.432011 65.339989) (end 142.748 65.024) (width 0.4) (layer B.Cu) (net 12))
 (segment (start 142.748 61.976) (end 142.432011 61.660011) (width 0.4) (layer B.Cu) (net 12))
 (segment (start 142.432011 61.660011) (end 137.632046 61.660011) (width 0.4) (layer B.Cu) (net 12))
 (segment (start 135.951989 59.979954) (end 135.951989 57.368046) (width 0.4) (layer B.Cu) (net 12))
 (segment (start 142.748 65.024) (end 142.748 61.976) (width 0.4) (layer B.Cu) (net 12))
 (segment (start 137.632046 61.660011) (end 135.951989 59.979954) (width 0.4) (layer B.Cu) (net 12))
 (segment (start 137.378046 55.941989) (end 161.912059 55.941989) (width 0.4) (layer B.Cu) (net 12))
 (segment (start 177.038 55.245) (end 178.435 55.245) (width 0.4) (layer B.Cu) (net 12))
 (segment (start 161.912059 55.941989) (end 162.302125 56.332055) (width 0.4) (layer B.Cu) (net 12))
 (segment (start 162.302125 56.332055) (end 175.950945 56.332055) (width 0.4) (layer B.Cu) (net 12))
 (segment (start 175.950945 56.332055) (end 177.038 55.245) (width 0.4) (layer B.Cu) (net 12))
 (segment (start 178.435 55.245) (end 181.864001 51.815999) (width 0.4) (layer B.Cu) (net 12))
 (segment (start 181.864001 51.815999) (end 182.88 50.8) (width 0.4) (layer B.Cu) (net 12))
 (segment (start 139.184001 71.755) (end 144.402022 66.536979) (width 0.4) (layer B.Cu) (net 13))
 (segment (start 167.132 42.164) (end 166.243 41.275) (width 0.4) (layer B.Cu) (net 13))
 (segment (start 54.737 56.007) (end 52.451 58.293) (width 0.4) (layer B.Cu) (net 13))
 (segment (start 156.337 49.022) (end 66.167 49.022) (width 0.4) (layer B.Cu) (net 13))
 (segment (start 52.451 58.293) (end 52.451 69.215) (width 0.4) (layer B.Cu) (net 13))
 (segment (start 54.991 71.755) (end 139.184001 71.755) (width 0.4) (layer B.Cu) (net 13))
 (segment (start 144.402022 66.536979) (end 144.402022 61.650092) (width 0.4) (layer B.Cu) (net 13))
 (segment (start 144.402022 61.650092) (end 141.55293 58.801) (width 0.4) (layer B.Cu) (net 13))
 (segment (start 167.64 43.18) (end 167.132 42.672) (width 0.4) (layer B.Cu) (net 13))
 (segment (start 167.132 42.672) (end 167.132 42.164) (width 0.4) (layer B.Cu) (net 13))
 (segment (start 66.167 49.022) (end 59.182 56.007) (width 0.4) (layer B.Cu) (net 13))
 (segment (start 166.243 41.275) (end 164.084 41.275) (width 0.4) (layer B.Cu) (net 13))
 (segment (start 164.084 41.275) (end 156.337 49.022) (width 0.4) (layer B.Cu) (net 13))
 (segment (start 59.182 56.007) (end 54.737 56.007) (width 0.4) (layer B.Cu) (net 13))
 (segment (start 52.451 69.215) (end 54.991 71.755) (width 0.4) (layer B.Cu) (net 13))
 (segment (start 141.55293 58.801) (end 139.7 58.801) (width 0.4) (layer B.Cu) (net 13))
 (segment (start 53.151011 58.582953) (end 54.964964 56.769) (width 0.4) (layer B.Cu) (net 14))
 (segment (start 54.964964 56.769) (end 59.436 56.769) (width 0.4) (layer B.Cu) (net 14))
 (segment (start 59.436 56.769) (end 66.482989 49.722011) (width 0.4) (layer B.Cu) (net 14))
 (segment (start 163.66316 43.18) (end 165.1 43.18) (width 0.4) (layer B.Cu) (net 14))
 (segment (start 156.626954 49.722011) (end 163.168965 43.18) (width 0.4) (layer B.Cu) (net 14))
 (segment (start 55.333024 71.054989) (end 53.151011 68.872976) (width 0.4) (layer B.Cu) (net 14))
 (segment (start 66.482989 49.722011) (end 156.626954 49.722011) (width 0.4) (layer B.Cu) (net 14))
 (segment (start 163.168965 43.18) (end 163.66316 43.18) (width 0.4) (layer B.Cu) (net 14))
 (segment (start 53.151011 68.872976) (end 53.151011 58.582953) (width 0.4) (layer B.Cu) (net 14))
 (segment (start 139.7 68.199) (end 136.844011 71.054989) (width 0.4) (layer B.Cu) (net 14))
 (segment (start 136.844011 71.054989) (end 55.333024 71.054989) (width 0.4) (layer B.Cu) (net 14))
 (segment (start 160.42 58.801) (end 158.75 58.801) (width 0.4) (layer B.Cu) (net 15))
 (segment (start 212.887953 70.292989) (end 177.274387 70.292989) (width 0.4) (layer B.Cu) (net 15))
 (segment (start 165.782398 58.801) (end 160.42 58.801) (width 0.4) (layer B.Cu) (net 15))
 (segment (start 177.274387 70.292989) (end 165.782398 58.801) (width 0.4) (layer B.Cu) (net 15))
 (segment (start 213.968962 71.374) (end 212.887953 70.292989) (width 0.4) (layer B.Cu) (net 15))
 (segment (start 217.450038 71.374) (end 213.968962 71.374) (width 0.4) (layer B.Cu) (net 15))
 (segment (start 221.676989 67.147049) (end 217.450038 71.374) (width 0.4) (layer B.Cu) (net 15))
 (segment (start 221.676989 47.664129) (end 221.676989 67.147049) (width 0.4) (layer B.Cu) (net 15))
 (segment (start 211.787805 37.774945) (end 221.676989 47.664129) (width 0.4) (layer B.Cu) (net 15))
 (segment (start 172.72 43.18) (end 178.125055 37.774945) (width 0.4) (layer B.Cu) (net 15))
 (segment (start 178.125055 37.774945) (end 211.787805 37.774945) (width 0.4) (layer B.Cu) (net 15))
 (segment (start 217.739992 72.074011) (end 213.679008 72.074011) (width 0.4) (layer B.Cu) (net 16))
 (segment (start 160.019999 69.468999) (end 158.75 68.199) (width 0.4) (layer B.Cu) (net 16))
 (segment (start 213.679008 72.074011) (end 212.598 70.993) (width 0.4) (layer B.Cu) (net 16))
 (segment (start 212.080934 37.074934) (end 222.377 47.371) (width 0.4) (layer B.Cu) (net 16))
 (segment (start 222.377 47.371) (end 222.377 67.437003) (width 0.4) (layer B.Cu) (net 16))
 (segment (start 176.285066 37.074934) (end 212.080934 37.074934) (width 0.4) (layer B.Cu) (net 16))
 (segment (start 161.544 70.993) (end 160.019999 69.468999) (width 0.4) (layer B.Cu) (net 16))
 (segment (start 170.18 43.18) (end 176.285066 37.074934) (width 0.4) (layer B.Cu) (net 16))
 (segment (start 222.377 67.437003) (end 217.739992 72.074011) (width 0.4) (layer B.Cu) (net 16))
 (segment (start 212.598 70.993) (end 161.544 70.993) (width 0.4) (layer B.Cu) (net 16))
 (segment (start 203.375895 58.801) (end 179.47 58.801) (width 0.4) (layer B.Cu) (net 17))
 (segment (start 211.207897 39.174967) (end 220.276967 48.244037) (width 0.4) (layer B.Cu) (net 17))
 (segment (start 191.526072 39.184033) (end 191.535138 39.174967) (width 0.4) (layer B.Cu) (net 17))
 (segment (start 179.47 58.801) (end 177.8 58.801) (width 0.4) (layer B.Cu) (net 17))
 (segment (start 213.467862 68.892967) (end 203.375895 58.801) (width 0.4) (layer B.Cu) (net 17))
 (segment (start 214.54887 69.973978) (end 213.467862 68.892967) (width 0.4) (layer B.Cu) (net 17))
 (segment (start 220.276967 48.244037) (end 220.276967 66.567141) (width 0.4) (layer B.Cu) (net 17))
 (segment (start 220.276967 66.567141) (end 216.87013 69.973978) (width 0.4) (layer B.Cu) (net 17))
 (segment (start 191.535138 39.174967) (end 211.207897 39.174967) (width 0.4) (layer B.Cu) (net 17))
 (segment (start 216.87013 69.973978) (end 214.54887 69.973978) (width 0.4) (layer B.Cu) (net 17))
 (segment (start 181.795967 39.184033) (end 191.526072 39.184033) (width 0.4) (layer B.Cu) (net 17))
 (segment (start 177.8 43.18) (end 181.795967 39.184033) (width 0.4) (layer B.Cu) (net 17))
 (segment (start 176.275999 42.164001) (end 175.26 43.18) (width 0.4) (layer B.Cu) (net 18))
 (segment (start 191.245184 38.474956) (end 191.236118 38.484022) (width 0.4) (layer B.Cu) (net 18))
 (segment (start 179.955978 38.484022) (end 176.275999 42.164001) (width 0.4) (layer B.Cu) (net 18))
 (segment (start 220.976978 47.954083) (end 211.497851 38.474956) (width 0.4) (layer B.Cu) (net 18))
 (segment (start 211.497851 38.474956) (end 191.245184 38.474956) (width 0.4) (layer B.Cu) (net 18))
 (segment (start 211.783928 68.199) (end 214.258916 70.673989) (width 0.4) (layer B.Cu) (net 18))
 (segment (start 220.976978 66.857095) (end 220.976978 47.954083) (width 0.4) (layer B.Cu) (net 18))
 (segment (start 217.160084 70.673989) (end 220.976978 66.857095) (width 0.4) (layer B.Cu) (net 18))
 (segment (start 177.8 68.199) (end 211.783928 68.199) (width 0.4) (layer B.Cu) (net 18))
 (segment (start 214.258916 70.673989) (end 217.160084 70.673989) (width 0.4) (layer B.Cu) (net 18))
 (segment (start 191.236118 38.484022) (end 179.955978 38.484022) (width 0.4) (layer B.Cu) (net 18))
 (segment (start 215.9 58.801) (end 215.9 45.847) (width 0.4) (layer B.Cu) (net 19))
 (segment (start 192.115046 40.574989) (end 192.10598 40.584055) (width 0.4) (layer B.Cu) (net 19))
 (segment (start 210.627989 40.574989) (end 192.115046 40.574989) (width 0.4) (layer B.Cu) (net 19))
 (segment (start 192.10598 40.584055) (end 185.475945 40.584055) (width 0.4) (layer B.Cu) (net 19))
 (segment (start 215.9 45.847) (end 210.627989 40.574989) (width 0.4) (layer B.Cu) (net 19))
 (segment (start 183.895999 42.164001) (end 182.88 43.18) (width 0.4) (layer B.Cu) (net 19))
 (segment (start 185.475945 40.584055) (end 183.895999 42.164001) (width 0.4) (layer B.Cu) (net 19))
 (segment (start 191.825092 39.874978) (end 191.816026 39.884044) (width 0.4) (layer B.Cu) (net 20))
 (segment (start 191.816026 39.884044) (end 183.635956 39.884044) (width 0.4) (layer B.Cu) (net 20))
 (segment (start 219.576956 48.533991) (end 210.917943 39.874978) (width 0.4) (layer B.Cu) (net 20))
 (segment (start 219.576956 64.522044) (end 219.576956 48.533991) (width 0.4) (layer B.Cu) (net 20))
 (segment (start 215.9 68.199) (end 219.576956 64.522044) (width 0.4) (layer B.Cu) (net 20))
 (segment (start 183.635956 39.884044) (end 181.355999 42.164001) (width 0.4) (layer B.Cu) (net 20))
 (segment (start 210.917943 39.874978) (end 191.825092 39.874978) (width 0.4) (layer B.Cu) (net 20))
 (segment (start 181.355999 42.164001) (end 180.34 43.18) (width 0.4) (layer B.Cu) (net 20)))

